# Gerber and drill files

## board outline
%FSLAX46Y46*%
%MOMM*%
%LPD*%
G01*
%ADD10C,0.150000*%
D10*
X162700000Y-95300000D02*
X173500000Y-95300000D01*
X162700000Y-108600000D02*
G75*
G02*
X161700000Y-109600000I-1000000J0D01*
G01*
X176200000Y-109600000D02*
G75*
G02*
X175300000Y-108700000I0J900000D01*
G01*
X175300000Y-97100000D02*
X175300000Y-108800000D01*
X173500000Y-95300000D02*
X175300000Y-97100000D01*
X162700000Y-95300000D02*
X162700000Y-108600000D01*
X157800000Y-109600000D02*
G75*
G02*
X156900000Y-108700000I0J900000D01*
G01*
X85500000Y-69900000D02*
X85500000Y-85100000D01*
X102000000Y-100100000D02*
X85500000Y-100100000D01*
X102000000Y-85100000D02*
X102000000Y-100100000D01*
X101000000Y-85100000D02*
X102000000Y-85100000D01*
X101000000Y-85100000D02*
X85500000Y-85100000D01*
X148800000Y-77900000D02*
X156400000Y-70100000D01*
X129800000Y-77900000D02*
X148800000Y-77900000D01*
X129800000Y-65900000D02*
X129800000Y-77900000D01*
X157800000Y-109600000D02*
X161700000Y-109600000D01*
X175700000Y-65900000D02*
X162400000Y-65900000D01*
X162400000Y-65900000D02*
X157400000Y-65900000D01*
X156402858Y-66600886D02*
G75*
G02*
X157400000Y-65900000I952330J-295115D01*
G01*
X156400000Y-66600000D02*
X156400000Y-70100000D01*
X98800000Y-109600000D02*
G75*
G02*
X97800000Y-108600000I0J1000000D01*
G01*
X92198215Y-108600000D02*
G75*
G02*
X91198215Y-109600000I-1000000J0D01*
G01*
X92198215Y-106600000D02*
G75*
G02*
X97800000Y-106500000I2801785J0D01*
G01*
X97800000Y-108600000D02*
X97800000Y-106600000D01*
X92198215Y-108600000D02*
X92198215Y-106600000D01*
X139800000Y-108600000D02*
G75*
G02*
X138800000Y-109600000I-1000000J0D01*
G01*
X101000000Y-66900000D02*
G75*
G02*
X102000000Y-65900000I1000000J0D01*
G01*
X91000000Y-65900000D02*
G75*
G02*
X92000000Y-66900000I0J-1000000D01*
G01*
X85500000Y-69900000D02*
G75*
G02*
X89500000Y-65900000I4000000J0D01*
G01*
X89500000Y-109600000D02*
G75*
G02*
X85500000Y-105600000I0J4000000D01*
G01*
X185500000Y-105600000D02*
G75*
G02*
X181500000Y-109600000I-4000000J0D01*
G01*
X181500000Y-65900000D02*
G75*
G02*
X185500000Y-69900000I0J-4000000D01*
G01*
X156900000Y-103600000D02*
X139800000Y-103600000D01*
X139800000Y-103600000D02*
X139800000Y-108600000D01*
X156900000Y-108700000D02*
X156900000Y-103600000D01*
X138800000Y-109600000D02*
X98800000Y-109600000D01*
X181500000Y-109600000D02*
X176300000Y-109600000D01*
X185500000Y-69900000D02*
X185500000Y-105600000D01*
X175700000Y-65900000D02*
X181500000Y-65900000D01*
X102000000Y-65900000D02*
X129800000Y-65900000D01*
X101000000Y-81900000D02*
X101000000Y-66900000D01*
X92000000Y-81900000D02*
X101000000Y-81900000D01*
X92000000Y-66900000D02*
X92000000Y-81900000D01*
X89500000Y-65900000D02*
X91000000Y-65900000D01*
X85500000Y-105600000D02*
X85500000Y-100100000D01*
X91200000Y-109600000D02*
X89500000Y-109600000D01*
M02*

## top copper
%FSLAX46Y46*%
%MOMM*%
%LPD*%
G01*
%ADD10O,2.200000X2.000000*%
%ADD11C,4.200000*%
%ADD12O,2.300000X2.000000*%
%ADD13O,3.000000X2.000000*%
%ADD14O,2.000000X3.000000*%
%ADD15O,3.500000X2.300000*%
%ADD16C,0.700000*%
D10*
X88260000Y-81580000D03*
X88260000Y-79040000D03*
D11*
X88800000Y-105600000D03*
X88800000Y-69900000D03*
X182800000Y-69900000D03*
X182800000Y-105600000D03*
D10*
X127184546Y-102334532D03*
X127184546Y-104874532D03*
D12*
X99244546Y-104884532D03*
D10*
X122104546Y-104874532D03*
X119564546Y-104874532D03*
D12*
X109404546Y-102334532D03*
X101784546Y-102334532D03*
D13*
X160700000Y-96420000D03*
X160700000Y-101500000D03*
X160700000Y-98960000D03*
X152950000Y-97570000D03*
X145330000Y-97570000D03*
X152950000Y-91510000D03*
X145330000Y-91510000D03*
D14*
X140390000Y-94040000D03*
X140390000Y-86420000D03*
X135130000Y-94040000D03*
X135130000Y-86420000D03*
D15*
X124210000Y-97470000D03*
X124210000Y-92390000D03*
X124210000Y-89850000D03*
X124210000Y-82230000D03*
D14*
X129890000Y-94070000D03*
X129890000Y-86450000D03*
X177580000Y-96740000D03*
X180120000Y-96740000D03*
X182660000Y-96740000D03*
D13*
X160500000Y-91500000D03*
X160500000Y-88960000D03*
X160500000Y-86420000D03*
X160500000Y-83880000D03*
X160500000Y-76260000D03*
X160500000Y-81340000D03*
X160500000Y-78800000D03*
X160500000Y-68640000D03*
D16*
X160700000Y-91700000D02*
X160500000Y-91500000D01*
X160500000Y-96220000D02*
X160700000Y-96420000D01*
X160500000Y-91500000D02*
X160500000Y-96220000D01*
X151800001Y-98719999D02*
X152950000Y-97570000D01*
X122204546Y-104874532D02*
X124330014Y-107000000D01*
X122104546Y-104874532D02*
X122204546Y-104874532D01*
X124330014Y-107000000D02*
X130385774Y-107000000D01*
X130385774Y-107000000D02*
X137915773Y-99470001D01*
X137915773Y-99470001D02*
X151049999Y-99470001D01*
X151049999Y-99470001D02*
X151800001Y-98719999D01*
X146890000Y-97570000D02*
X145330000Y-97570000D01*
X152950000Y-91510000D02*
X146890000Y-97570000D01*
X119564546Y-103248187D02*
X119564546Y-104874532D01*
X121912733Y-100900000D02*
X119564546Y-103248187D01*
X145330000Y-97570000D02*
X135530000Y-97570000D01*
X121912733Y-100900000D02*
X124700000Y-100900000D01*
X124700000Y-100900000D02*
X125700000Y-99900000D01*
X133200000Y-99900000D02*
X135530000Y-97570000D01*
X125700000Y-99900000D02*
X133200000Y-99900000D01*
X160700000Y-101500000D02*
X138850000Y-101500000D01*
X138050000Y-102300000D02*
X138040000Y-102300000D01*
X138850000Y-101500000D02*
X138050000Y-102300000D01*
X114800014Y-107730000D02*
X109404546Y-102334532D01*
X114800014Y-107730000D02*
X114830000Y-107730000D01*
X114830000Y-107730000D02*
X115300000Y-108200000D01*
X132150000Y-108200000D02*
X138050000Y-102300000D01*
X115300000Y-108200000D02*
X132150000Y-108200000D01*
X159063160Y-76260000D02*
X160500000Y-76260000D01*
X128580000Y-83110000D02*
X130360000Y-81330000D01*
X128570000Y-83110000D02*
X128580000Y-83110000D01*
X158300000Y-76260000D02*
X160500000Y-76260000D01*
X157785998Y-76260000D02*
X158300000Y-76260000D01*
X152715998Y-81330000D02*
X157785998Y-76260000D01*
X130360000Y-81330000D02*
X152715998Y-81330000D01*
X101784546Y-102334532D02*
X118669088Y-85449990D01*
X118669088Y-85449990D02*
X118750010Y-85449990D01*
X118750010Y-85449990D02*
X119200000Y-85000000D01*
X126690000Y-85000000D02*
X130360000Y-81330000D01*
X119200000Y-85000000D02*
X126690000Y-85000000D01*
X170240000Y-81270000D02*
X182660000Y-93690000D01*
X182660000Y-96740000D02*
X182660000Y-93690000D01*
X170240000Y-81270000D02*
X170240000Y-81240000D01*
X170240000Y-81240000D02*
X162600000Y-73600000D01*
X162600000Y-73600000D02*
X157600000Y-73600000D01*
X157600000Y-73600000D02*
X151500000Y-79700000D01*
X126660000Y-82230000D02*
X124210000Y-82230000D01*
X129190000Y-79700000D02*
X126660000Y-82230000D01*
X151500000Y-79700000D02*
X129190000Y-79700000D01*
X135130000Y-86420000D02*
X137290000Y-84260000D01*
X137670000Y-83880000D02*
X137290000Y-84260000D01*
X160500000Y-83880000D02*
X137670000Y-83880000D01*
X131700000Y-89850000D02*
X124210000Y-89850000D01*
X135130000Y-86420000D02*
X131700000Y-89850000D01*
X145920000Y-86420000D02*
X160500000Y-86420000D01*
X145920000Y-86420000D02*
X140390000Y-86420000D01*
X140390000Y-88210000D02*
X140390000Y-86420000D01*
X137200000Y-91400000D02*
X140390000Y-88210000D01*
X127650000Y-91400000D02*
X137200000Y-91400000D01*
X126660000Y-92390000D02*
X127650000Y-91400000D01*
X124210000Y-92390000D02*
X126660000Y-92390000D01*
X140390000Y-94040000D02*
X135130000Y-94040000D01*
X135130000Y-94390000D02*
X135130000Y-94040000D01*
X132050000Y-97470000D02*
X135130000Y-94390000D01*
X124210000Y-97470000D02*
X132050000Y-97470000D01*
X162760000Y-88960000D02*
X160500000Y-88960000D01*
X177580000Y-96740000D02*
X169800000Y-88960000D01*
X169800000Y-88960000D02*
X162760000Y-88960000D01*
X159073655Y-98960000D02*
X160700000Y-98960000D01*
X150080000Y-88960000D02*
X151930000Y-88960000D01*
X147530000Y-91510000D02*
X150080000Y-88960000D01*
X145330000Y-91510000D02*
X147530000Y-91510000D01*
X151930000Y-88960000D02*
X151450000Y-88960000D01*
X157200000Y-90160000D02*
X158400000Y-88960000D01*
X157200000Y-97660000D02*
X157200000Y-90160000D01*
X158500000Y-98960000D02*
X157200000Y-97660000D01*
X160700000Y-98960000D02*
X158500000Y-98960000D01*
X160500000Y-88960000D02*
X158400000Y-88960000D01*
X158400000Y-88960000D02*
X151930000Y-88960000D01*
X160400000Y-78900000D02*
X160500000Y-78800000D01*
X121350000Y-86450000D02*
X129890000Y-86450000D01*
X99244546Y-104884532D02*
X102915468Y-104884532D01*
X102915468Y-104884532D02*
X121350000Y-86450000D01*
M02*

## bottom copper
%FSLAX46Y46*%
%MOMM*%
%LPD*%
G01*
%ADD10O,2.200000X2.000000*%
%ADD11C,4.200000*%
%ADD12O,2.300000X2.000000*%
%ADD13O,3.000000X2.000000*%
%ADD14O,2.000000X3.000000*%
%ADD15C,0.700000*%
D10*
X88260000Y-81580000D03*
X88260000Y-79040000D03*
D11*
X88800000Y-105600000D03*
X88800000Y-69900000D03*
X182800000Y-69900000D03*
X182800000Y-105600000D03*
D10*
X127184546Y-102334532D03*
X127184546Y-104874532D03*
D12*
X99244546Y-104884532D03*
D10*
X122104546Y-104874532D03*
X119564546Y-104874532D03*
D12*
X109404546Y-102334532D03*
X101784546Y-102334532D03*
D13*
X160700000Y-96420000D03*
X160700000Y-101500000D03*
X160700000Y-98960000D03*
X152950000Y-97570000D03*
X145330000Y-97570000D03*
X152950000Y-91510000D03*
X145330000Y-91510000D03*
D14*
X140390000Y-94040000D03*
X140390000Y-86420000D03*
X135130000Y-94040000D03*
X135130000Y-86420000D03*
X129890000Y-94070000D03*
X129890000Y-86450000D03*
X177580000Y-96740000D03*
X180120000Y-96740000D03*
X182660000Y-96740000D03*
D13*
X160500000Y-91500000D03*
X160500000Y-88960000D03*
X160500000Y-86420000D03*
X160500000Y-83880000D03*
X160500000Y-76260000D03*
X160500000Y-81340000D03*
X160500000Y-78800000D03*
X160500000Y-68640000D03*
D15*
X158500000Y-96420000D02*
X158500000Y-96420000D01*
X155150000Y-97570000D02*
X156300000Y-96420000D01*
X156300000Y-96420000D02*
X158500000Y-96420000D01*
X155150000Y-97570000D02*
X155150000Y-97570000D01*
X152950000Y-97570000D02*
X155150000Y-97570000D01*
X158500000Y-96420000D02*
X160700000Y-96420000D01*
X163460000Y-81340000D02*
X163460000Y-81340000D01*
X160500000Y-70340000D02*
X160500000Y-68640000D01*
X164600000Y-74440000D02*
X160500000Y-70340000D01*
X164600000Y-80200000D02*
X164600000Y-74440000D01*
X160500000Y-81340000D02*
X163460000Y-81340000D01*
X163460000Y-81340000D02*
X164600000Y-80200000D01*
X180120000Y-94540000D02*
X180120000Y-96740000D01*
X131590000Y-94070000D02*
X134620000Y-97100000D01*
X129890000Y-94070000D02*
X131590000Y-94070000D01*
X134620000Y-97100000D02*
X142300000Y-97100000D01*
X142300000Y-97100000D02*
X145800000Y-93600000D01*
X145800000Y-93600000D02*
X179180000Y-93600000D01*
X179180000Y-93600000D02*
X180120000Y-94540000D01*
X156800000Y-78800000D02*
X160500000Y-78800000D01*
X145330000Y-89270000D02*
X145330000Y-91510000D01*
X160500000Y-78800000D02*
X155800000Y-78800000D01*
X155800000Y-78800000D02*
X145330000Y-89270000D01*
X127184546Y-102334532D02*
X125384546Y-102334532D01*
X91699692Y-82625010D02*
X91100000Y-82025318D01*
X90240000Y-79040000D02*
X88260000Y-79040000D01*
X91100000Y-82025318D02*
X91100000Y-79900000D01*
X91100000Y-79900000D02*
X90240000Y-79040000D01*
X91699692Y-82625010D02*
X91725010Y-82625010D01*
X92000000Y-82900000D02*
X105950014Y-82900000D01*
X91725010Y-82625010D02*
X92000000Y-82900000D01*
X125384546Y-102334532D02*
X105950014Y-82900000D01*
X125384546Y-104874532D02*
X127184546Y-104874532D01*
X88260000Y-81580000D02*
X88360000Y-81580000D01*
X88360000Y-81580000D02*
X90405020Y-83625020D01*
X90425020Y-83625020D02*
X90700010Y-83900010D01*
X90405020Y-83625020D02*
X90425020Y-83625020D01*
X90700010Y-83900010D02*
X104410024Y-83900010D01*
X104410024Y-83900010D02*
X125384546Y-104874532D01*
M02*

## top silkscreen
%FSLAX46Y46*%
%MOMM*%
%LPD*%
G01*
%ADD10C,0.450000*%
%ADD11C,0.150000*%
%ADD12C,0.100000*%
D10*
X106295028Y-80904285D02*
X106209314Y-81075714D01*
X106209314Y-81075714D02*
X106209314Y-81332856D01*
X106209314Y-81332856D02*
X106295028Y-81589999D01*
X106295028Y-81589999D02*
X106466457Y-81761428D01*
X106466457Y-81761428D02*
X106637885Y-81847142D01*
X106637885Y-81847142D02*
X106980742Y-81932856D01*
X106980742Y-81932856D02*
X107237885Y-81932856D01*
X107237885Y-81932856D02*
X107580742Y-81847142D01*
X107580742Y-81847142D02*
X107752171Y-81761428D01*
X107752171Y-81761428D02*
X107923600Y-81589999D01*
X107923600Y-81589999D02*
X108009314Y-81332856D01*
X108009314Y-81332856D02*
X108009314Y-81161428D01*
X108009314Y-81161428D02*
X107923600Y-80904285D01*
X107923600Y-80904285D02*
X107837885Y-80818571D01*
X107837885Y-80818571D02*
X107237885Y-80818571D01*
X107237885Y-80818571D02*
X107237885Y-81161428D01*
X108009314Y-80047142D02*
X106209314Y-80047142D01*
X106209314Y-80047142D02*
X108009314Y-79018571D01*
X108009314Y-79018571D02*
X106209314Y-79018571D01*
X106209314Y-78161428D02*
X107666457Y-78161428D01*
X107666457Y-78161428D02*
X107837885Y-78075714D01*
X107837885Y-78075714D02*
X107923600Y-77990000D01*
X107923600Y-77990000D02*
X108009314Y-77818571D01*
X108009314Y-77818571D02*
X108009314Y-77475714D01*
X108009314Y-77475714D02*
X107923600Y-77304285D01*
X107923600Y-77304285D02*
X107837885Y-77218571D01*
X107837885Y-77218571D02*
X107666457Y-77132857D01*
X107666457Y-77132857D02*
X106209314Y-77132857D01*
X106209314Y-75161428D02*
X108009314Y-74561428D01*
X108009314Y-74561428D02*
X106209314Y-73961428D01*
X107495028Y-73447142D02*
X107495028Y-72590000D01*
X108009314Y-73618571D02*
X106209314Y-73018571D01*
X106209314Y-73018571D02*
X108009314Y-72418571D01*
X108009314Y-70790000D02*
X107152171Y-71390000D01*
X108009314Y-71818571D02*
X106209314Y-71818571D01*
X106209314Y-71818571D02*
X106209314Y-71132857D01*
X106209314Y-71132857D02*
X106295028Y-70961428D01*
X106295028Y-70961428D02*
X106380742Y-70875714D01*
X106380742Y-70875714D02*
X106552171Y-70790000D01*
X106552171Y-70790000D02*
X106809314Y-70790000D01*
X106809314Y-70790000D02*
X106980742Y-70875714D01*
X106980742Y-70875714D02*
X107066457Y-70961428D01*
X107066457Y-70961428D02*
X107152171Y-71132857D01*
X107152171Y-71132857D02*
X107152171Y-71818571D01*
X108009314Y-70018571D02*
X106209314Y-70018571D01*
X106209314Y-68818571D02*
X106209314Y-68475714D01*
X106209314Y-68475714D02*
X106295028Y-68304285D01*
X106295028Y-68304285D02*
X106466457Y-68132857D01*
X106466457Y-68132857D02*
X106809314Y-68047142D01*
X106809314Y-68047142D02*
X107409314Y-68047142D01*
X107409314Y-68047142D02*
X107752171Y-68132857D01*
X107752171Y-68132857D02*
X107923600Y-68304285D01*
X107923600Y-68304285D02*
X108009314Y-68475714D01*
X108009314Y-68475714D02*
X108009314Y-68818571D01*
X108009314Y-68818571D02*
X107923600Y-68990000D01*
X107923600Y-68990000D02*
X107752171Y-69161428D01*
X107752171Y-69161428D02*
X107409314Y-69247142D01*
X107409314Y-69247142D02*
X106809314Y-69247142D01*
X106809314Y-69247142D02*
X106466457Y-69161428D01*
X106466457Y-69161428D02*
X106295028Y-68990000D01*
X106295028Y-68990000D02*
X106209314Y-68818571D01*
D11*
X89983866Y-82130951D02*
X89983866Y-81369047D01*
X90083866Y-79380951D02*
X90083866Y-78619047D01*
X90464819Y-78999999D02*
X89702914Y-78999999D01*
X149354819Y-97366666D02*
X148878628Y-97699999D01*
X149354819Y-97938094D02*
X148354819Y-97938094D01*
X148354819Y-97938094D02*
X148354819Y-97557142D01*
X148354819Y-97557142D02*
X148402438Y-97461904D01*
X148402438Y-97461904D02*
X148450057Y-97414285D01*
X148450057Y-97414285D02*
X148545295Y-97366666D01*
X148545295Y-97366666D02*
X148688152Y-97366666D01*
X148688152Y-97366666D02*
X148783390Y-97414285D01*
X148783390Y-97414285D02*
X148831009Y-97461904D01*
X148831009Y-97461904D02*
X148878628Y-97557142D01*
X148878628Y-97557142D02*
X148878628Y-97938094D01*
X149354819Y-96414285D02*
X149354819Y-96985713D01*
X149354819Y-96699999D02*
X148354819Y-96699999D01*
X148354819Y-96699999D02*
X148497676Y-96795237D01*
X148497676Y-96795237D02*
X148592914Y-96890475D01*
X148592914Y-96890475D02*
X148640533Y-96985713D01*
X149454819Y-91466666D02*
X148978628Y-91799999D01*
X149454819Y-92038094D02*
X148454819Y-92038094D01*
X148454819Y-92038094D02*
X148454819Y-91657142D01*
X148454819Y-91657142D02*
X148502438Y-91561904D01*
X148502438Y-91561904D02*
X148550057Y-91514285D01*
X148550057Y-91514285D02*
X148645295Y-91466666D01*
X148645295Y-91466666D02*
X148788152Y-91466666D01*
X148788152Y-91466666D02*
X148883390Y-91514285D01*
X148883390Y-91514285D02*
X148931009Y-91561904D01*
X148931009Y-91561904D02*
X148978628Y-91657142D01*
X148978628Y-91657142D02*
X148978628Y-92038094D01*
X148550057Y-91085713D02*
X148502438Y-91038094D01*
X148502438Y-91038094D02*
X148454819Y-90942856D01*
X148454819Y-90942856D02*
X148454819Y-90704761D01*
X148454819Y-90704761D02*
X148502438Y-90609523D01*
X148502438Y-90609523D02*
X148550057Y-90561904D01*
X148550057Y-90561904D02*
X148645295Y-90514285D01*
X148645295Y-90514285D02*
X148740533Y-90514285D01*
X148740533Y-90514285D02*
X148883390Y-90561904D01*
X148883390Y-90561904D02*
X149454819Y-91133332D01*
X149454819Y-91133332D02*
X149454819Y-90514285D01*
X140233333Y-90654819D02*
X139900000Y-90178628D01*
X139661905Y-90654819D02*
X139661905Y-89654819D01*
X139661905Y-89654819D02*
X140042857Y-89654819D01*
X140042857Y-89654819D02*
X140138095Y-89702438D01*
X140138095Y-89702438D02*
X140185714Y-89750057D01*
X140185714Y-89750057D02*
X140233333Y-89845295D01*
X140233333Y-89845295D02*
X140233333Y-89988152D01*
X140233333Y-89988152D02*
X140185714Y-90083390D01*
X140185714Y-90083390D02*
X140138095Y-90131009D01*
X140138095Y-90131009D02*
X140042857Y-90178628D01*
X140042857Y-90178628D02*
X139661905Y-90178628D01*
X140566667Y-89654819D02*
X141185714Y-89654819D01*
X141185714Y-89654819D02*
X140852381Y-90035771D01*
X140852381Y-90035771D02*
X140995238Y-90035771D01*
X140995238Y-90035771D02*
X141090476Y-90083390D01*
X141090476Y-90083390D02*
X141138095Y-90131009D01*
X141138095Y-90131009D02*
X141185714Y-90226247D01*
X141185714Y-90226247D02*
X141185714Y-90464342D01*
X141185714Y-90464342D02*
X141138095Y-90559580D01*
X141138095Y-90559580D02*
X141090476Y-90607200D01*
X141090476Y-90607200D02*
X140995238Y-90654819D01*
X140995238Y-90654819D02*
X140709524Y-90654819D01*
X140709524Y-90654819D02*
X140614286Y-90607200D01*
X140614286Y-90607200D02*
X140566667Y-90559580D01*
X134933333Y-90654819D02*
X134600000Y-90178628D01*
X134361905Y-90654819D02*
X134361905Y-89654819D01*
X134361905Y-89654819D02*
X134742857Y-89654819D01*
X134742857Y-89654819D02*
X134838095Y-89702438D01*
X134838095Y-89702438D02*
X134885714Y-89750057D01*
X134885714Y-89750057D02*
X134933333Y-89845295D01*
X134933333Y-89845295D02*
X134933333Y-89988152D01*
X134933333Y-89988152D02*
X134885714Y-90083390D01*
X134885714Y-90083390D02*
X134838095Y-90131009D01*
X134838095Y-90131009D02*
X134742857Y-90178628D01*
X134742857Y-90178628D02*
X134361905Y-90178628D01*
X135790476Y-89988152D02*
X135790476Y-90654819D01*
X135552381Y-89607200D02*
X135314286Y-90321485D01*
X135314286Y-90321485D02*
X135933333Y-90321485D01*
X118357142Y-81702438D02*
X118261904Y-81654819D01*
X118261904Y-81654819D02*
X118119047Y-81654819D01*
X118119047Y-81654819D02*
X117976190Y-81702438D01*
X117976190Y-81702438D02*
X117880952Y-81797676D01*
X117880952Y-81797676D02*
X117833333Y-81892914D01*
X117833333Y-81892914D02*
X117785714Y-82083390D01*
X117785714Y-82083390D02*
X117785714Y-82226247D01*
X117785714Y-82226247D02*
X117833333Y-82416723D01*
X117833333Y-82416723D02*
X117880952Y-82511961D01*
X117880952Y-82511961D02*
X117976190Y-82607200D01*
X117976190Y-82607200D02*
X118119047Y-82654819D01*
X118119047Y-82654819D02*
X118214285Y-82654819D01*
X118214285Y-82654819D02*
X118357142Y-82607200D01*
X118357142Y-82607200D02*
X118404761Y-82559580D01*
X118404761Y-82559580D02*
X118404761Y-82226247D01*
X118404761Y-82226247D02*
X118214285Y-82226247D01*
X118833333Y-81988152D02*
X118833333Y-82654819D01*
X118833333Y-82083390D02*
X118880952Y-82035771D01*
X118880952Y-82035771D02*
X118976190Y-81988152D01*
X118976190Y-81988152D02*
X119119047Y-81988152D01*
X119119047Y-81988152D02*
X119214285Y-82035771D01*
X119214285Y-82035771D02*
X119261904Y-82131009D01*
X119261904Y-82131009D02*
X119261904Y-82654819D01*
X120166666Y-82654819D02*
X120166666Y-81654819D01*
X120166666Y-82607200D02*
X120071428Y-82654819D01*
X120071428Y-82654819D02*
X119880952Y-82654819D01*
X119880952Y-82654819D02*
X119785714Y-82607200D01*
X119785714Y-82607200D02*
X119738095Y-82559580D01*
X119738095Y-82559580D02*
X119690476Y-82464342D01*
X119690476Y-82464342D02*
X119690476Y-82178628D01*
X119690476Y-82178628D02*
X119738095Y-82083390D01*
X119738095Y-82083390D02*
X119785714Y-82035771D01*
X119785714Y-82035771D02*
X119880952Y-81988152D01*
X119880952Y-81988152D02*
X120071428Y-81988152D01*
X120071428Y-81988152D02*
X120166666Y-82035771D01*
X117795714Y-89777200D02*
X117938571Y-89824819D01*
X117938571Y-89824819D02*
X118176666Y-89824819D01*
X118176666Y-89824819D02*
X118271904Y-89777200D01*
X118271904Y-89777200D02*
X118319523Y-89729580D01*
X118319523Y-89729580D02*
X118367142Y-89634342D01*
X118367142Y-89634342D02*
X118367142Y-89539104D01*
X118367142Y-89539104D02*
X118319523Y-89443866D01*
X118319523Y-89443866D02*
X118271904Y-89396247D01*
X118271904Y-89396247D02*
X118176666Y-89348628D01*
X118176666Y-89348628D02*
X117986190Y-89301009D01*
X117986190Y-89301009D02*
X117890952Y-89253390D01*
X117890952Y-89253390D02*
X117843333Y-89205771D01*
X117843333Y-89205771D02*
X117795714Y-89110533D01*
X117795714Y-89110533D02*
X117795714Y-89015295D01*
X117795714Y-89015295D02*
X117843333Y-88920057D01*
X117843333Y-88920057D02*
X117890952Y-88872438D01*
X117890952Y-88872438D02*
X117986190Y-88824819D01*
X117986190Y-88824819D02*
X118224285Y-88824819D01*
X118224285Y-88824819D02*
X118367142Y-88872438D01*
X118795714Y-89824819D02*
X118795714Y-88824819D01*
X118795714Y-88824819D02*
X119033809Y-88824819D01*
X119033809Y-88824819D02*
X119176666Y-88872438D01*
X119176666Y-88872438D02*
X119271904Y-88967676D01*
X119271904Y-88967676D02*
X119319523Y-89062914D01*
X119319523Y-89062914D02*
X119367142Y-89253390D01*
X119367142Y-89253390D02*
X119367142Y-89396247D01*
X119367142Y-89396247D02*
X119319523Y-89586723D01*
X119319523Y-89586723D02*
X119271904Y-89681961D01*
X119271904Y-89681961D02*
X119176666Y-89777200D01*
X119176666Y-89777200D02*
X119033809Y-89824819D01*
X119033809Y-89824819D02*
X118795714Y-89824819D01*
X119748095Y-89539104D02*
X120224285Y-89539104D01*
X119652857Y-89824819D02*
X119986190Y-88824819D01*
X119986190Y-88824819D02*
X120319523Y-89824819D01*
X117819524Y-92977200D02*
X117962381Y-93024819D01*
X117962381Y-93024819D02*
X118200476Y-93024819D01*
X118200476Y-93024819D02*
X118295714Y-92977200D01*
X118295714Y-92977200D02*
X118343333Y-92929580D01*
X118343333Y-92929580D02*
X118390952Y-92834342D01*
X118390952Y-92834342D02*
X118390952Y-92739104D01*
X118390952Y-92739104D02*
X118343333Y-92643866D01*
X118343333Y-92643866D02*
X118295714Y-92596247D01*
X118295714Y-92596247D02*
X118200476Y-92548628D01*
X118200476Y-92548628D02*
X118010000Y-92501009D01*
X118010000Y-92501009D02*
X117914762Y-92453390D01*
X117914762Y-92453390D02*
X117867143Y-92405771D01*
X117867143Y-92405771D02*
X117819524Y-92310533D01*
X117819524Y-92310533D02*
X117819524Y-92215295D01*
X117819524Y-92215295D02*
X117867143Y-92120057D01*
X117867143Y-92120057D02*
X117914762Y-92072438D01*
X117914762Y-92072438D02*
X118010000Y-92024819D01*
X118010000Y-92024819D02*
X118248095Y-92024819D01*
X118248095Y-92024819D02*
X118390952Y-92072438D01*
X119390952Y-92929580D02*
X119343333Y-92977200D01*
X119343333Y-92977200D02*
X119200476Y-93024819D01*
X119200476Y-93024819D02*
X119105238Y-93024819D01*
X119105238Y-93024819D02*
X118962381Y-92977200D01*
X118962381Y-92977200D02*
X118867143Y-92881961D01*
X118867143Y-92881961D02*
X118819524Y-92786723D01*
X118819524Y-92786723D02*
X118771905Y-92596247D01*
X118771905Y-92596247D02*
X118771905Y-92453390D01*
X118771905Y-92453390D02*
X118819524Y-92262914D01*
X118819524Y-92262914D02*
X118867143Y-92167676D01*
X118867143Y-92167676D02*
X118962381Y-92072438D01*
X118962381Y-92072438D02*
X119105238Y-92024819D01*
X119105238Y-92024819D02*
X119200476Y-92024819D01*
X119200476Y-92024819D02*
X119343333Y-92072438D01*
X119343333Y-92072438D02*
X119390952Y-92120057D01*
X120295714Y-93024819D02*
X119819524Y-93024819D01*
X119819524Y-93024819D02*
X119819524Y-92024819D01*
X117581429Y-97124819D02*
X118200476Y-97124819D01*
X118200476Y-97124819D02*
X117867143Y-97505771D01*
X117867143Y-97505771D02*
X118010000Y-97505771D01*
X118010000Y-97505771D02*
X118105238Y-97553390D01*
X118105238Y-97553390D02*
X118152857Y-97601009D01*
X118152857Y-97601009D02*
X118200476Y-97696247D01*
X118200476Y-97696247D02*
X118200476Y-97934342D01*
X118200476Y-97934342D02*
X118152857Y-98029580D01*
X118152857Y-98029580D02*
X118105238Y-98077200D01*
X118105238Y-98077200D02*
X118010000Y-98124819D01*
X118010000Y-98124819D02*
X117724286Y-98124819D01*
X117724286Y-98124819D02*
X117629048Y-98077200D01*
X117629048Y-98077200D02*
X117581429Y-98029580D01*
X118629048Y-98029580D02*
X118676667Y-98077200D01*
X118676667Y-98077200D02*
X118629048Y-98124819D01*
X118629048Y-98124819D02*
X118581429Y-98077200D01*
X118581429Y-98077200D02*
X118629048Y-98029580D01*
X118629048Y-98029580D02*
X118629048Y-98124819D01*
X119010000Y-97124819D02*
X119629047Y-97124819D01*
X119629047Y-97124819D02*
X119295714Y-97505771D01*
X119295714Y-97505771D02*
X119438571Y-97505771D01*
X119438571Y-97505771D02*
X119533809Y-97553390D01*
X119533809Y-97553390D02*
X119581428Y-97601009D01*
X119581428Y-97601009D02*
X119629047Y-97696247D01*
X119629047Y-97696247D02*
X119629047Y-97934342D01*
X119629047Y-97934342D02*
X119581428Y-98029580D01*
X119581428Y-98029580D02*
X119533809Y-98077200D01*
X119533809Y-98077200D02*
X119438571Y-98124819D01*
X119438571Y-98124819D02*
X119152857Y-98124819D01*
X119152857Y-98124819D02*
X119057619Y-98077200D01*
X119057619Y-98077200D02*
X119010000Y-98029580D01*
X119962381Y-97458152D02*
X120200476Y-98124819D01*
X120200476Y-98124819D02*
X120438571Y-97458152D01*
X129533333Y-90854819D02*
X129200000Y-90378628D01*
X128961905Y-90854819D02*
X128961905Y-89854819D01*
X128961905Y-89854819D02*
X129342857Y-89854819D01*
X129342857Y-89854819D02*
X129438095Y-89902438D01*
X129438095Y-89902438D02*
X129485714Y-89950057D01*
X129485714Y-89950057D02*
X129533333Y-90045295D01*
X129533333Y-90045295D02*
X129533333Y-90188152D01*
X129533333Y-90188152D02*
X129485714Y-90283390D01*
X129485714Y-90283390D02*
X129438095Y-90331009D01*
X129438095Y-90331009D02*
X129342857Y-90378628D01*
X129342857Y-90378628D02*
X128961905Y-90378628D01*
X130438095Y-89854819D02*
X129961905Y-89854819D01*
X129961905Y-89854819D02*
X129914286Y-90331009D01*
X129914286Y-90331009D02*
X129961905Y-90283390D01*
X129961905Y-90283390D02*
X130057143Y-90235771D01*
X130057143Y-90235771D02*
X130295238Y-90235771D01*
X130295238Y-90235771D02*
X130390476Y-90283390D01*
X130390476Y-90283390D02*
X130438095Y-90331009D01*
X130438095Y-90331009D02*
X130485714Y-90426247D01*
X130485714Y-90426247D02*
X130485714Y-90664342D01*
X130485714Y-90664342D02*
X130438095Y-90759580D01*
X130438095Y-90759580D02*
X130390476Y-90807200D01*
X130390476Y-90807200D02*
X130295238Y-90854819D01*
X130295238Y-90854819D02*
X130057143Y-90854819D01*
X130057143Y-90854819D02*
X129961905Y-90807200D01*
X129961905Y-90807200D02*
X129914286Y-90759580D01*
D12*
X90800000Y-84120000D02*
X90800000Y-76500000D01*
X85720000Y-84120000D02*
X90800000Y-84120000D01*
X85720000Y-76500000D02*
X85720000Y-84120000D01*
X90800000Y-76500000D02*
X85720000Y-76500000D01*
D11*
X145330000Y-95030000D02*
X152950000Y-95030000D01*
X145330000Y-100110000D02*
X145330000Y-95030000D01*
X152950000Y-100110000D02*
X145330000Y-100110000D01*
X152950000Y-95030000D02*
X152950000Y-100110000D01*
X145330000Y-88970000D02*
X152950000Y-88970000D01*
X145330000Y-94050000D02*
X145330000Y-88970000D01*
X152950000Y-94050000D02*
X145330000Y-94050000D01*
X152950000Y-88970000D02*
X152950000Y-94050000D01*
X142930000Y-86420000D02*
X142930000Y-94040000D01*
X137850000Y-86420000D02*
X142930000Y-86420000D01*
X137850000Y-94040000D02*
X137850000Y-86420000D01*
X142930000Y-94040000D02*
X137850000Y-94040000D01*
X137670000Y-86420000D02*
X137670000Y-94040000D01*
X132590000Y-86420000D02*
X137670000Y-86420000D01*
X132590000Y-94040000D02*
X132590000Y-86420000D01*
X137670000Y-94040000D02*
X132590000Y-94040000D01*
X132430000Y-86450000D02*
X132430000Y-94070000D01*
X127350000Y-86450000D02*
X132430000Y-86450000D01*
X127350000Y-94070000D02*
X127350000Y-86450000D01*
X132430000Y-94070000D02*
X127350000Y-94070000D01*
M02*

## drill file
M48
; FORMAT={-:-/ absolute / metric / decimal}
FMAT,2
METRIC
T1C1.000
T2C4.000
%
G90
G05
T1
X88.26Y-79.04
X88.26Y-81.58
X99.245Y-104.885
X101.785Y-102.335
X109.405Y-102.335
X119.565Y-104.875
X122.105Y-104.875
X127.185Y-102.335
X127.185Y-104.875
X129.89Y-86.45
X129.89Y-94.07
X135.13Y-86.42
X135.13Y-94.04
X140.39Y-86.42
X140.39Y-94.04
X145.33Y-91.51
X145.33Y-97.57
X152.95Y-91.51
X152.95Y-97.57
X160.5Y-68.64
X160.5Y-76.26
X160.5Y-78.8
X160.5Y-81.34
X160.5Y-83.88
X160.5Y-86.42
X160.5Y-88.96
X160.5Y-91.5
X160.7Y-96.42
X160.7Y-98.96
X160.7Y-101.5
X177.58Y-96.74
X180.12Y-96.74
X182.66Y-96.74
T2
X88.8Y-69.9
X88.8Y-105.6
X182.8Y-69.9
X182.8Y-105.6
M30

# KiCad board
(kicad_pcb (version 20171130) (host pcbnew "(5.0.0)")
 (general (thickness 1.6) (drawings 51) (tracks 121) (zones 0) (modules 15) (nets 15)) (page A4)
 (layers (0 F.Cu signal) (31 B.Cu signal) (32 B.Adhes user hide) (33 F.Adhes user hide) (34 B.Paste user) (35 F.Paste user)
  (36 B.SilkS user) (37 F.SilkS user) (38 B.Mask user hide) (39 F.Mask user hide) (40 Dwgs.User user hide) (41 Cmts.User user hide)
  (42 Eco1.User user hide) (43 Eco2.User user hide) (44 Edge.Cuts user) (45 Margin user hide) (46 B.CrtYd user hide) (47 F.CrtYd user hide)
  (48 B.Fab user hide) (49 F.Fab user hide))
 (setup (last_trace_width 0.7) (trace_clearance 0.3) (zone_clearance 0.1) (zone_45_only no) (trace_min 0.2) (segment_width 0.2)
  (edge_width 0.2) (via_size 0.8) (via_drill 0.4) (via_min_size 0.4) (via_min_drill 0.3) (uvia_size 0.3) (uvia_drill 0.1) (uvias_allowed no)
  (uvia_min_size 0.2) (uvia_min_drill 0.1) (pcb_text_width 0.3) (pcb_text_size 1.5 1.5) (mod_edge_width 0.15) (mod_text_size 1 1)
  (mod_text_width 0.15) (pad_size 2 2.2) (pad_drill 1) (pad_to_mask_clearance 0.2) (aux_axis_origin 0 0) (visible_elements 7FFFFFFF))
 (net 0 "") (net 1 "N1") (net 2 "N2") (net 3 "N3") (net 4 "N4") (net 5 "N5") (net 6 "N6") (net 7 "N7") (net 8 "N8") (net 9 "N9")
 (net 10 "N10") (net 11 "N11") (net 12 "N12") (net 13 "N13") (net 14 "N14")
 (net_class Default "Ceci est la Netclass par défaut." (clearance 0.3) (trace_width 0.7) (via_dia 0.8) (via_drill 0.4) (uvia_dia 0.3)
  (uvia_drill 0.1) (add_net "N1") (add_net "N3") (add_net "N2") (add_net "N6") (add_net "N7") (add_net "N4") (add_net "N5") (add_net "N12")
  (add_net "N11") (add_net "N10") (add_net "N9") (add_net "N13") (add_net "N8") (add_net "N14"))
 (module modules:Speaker (layer B.Cu) (at 90.8 76.5 270)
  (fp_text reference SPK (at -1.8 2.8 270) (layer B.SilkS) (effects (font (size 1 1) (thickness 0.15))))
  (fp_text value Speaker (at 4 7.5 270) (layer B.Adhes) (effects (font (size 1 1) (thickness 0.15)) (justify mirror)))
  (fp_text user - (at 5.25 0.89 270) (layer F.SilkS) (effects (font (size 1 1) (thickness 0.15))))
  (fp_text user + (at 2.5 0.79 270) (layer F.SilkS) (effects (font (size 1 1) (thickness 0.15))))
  (fp_line (start 7.62 0) (end 0 0) (layer F.SilkS) (width 0.1))
  (fp_line (start 7.62 5.08) (end 7.62 0) (layer F.SilkS) (width 0.1))
  (fp_line (start 0 5.08) (end 7.62 5.08) (layer F.SilkS) (width 0.1))
  (fp_line (start 0 0) (end 0 5.08) (layer F.SilkS) (width 0.1))
  (pad 2 thru_hole oval (at 5.08 2.54 270) (size 2 2.2) (drill 1) (layers *.Cu *.Paste *.Mask) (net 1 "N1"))
  (pad 1 thru_hole oval (at 2.54 2.54 270) (size 2 2.2) (drill 1) (layers *.Cu *.Paste *.Mask) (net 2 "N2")))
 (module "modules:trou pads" (layer F.Cu) (at 88.8 105.6)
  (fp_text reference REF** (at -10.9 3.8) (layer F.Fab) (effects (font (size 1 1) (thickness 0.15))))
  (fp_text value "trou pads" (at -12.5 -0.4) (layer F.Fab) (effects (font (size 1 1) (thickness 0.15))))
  (pad "" np_thru_hole circle (at 0 0) (size 4.2 4.2) (drill 4) (layers *.Cu *.Mask)))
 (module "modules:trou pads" (layer F.Cu) (at 88.8 69.9)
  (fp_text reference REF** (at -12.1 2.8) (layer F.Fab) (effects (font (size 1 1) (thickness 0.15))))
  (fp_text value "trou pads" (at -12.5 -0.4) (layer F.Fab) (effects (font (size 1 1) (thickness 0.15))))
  (pad "" np_thru_hole circle (at 0 0) (size 4.2 4.2) (drill 4) (layers *.Cu *.Mask)))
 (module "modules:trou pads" (layer F.Cu) (at 182.8 69.9)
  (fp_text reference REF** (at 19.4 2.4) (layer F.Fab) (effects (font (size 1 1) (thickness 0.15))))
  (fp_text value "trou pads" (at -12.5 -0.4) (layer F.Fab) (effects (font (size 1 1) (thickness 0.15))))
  (pad "" np_thru_hole circle (at 0 0) (size 4.2 4.2) (drill 4) (layers *.Cu *.Mask)))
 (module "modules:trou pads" (layer F.Cu) (at 182.8 105.6)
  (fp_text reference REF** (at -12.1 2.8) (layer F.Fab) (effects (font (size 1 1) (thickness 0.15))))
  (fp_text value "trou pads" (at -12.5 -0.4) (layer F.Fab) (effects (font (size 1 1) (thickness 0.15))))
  (pad "" np_thru_hole circle (at 0 0) (size 4.2 4.2) (drill 4) (layers *.Cu *.Mask)))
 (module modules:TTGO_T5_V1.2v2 (layer F.Cu) (at 127.734546 102.554532 90)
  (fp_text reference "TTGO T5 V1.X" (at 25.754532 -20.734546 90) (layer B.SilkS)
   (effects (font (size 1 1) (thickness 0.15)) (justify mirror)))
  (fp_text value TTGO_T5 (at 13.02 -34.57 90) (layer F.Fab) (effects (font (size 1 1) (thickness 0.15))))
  (pad "HP +" thru_hole oval (at 0.22 -0.55 90) (size 2 2.2) (drill 1) (layers *.Cu *.Paste *.Mask) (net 2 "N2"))
  (pad "HP -" thru_hole oval (at -2.32 -0.55 90) (size 2 2.2) (drill 1) (layers *.Cu *.Paste *.Mask) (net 1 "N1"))
  (pad 12 thru_hole oval (at -2.33 -28.49 90) (size 2 2.3) (drill 1) (layers *.Cu *.Paste *.Mask) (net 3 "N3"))
  (pad 3 thru_hole oval (at -2.32 -5.63 90) (size 2 2.2) (drill 1) (layers *.Cu *.Paste *.Mask) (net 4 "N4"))
  (pad 4 thru_hole oval (at -2.32 -8.17 90) (size 2 2.2) (drill 1) (layers *.Cu *.Paste *.Mask) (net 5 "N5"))
  (pad 20 thru_hole oval (at 0.22 -18.33 90) (size 2 2.3) (drill 1) (layers *.Cu *.Paste *.Mask) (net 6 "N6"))
  (pad 23 thru_hole oval (at 0.22 -25.95 90) (size 2 2.3) (drill 1) (layers *.Cu *.Paste *.Mask) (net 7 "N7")))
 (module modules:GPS (layer F.Cu) (at 160.7 96.42 270)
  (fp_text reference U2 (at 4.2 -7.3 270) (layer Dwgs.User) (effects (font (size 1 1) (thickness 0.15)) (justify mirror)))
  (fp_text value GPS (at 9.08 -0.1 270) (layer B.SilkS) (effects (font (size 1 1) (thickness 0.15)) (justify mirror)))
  (pad 1 thru_hole oval (at 0 0 270) (size 2 3) (drill 1) (layers *.Cu *.Paste *.Mask) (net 4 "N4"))
  (pad 3 thru_hole oval (at 5.08 0 270) (size 2 3) (drill 1) (layers *.Cu *.Paste *.Mask) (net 6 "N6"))
  (pad 2 thru_hole oval (at 2.54 0 270) (size 2 3) (drill 1) (layers *.Cu *.Paste *.Mask) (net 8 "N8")))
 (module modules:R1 (layer F.Cu) (at 145.33 97.57 270)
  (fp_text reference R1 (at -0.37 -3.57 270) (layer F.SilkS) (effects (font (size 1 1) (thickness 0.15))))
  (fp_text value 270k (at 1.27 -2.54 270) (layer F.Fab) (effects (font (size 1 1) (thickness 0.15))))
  (fp_line (start -2.54 0) (end -2.54 -7.62) (layer F.SilkS) (width 0.15))
  (fp_line (start 2.54 0) (end -2.54 0) (layer F.SilkS) (width 0.15))
  (fp_line (start 2.54 -7.62) (end 2.54 0) (layer F.SilkS) (width 0.15))
  (fp_line (start -2.54 -7.62) (end 2.54 -7.62) (layer F.SilkS) (width 0.15))
  (pad 2 thru_hole oval (at 0 -7.62 270) (size 2 3) (drill 1) (layers *.Cu *.Paste *.Mask) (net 4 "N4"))
  (pad 1 thru_hole oval (at 0 0 270) (size 2 3) (drill 1) (layers *.Cu *.Paste *.Mask) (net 5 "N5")))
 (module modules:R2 (layer F.Cu) (at 145.33 91.51 270)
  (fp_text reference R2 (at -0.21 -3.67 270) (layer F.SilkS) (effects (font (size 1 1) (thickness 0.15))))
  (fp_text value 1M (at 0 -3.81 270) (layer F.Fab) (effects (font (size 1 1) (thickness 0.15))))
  (fp_line (start -2.54 0) (end -2.54 -7.62) (layer F.SilkS) (width 0.15))
  (fp_line (start 2.54 0) (end -2.54 0) (layer F.SilkS) (width 0.15))
  (fp_line (start 2.54 -7.62) (end 2.54 0) (layer F.SilkS) (width 0.15))
  (fp_line (start -2.54 -7.62) (end 2.54 -7.62) (layer F.SilkS) (width 0.15))
  (pad 2 thru_hole oval (at 0 -7.62 270) (size 2 3) (drill 1) (layers *.Cu *.Paste *.Mask) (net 5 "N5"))
  (pad 1 thru_hole oval (at 0 0 270) (size 2 3) (drill 1) (layers *.Cu *.Paste *.Mask) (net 8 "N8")))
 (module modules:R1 (layer F.Cu) (at 140.39 86.42 180)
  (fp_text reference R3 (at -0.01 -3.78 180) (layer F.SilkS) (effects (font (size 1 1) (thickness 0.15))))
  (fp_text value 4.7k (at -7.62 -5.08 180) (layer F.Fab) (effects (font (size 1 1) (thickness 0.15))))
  (fp_line (start -2.54 0) (end -2.54 -7.62) (layer F.SilkS) (width 0.15))
  (fp_line (start 2.54 0) (end -2.54 0) (layer F.SilkS) (width 0.15))
  (fp_line (start 2.54 -7.62) (end 2.54 0) (layer F.SilkS) (width 0.15))
  (fp_line (start -2.54 -7.62) (end 2.54 -7.62) (layer F.SilkS) (width 0.15))
  (pad 2 thru_hole oval (at 0 -7.62 180) (size 2 3) (drill 1) (layers *.Cu *.Paste *.Mask) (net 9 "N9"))
  (pad 1 thru_hole oval (at 0 0 180) (size 2 3) (drill 1) (layers *.Cu *.Paste *.Mask) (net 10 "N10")))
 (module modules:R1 (layer F.Cu) (at 135.13 86.42 180)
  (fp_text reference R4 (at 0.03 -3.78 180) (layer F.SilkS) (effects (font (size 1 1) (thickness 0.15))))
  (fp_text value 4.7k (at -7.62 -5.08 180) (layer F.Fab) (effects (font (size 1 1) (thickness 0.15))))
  (fp_line (start -2.54 0) (end -2.54 -7.62) (layer F.SilkS) (width 0.15))
  (fp_line (start 2.54 0) (end -2.54 0) (layer F.SilkS) (width 0.15))
  (fp_line (start 2.54 -7.62) (end 2.54 0) (layer F.SilkS) (width 0.15))
  (fp_line (start -2.54 -7.62) (end 2.54 -7.62) (layer F.SilkS) (width 0.15))
  (pad 2 thru_hole oval (at 0 -7.62 180) (size 2 3) (drill 1) (layers *.Cu *.Paste *.Mask) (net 9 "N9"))
  (pad 1 thru_hole oval (at 0 0 180) (size 2 3) (drill 1) (layers *.Cu *.Paste *.Mask) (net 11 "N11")))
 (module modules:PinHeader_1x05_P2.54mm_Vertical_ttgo (layer F.Cu) (at 124.21 84.77)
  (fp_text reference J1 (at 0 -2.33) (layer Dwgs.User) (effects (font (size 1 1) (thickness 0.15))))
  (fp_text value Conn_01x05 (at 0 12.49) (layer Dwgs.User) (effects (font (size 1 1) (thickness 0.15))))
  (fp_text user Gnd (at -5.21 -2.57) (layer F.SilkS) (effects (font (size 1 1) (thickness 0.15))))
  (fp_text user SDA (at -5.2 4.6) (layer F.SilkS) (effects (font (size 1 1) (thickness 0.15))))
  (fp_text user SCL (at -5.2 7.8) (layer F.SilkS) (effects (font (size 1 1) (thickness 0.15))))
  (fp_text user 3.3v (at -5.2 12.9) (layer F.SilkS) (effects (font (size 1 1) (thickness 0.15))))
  (pad 5 smd oval (at 0 12.7) (size 3.5 2.3) (layers F.Cu F.Paste F.Mask) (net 9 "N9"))
  (pad 4 smd oval (at 0 7.62) (size 3.5 2.3) (layers F.Cu F.Paste F.Mask) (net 10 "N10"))
  (pad 3 smd oval (at 0 5.08) (size 3.5 2.3) (layers F.Cu F.Paste F.Mask) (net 11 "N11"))
  (pad 1 smd oval (at 0 -2.54) (size 3.5 2.3) (layers F.Cu F.Paste F.Mask) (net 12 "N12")))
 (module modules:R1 (layer F.Cu) (at 129.89 86.45 180)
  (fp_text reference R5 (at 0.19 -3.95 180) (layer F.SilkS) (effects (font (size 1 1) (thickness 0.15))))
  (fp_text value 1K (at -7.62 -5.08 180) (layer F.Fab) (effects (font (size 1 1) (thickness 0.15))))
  (fp_line (start -2.54 0) (end -2.54 -7.62) (layer F.SilkS) (width 0.15))
  (fp_line (start 2.54 0) (end -2.54 0) (layer F.SilkS) (width 0.15))
  (fp_line (start 2.54 -7.62) (end 2.54 0) (layer F.SilkS) (width 0.15))
  (fp_line (start -2.54 -7.62) (end 2.54 -7.62) (layer F.SilkS) (width 0.15))
  (pad 2 thru_hole oval (at 0 -7.62 180) (size 2 3) (drill 1) (layers *.Cu *.Paste *.Mask) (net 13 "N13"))
  (pad 1 thru_hole oval (at 0 0 180) (size 2 3) (drill 1) (layers *.Cu *.Paste *.Mask) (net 3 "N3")))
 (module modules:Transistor (layer F.Cu) (at 185.2 94.2 180)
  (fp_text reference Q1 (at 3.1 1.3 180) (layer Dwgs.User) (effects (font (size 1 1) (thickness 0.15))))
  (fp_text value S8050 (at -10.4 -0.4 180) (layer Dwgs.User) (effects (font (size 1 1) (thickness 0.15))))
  (pad 3 thru_hole oval (at 7.62 -2.54 180) (size 2 3) (drill 1) (layers *.Cu *.Paste *.Mask) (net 8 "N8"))
  (pad 2 thru_hole oval (at 5.08 -2.54 180) (size 2 3) (drill 1) (layers *.Cu *.Paste *.Mask) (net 13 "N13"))
  (pad 1 thru_hole oval (at 2.54 -2.54 180) (size 2 3) (drill 1) (layers *.Cu *.Paste *.Mask) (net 12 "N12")))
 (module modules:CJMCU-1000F (layer B.Cu) (at 163.04 78.8 270)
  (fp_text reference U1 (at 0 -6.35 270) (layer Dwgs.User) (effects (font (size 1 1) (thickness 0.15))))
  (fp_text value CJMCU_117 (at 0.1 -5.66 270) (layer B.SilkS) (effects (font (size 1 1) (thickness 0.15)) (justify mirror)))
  (pad 1 thru_hole oval (at 12.7 2.54 270) (size 2 3) (drill 1) (layers *.Cu *.Paste *.Mask) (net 4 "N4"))
  (pad 2 thru_hole oval (at 10.16 2.54 270) (size 2 3) (drill 1) (layers *.Cu *.Paste *.Mask) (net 8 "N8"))
  (pad 3 thru_hole oval (at 7.62 2.54 270) (size 2 3) (drill 1) (layers *.Cu *.Paste *.Mask) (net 10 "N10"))
  (pad 4 thru_hole oval (at 5.08 2.54 270) (size 2 3) (drill 1) (layers *.Cu *.Paste *.Mask) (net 11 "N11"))
  (pad 7 thru_hole oval (at -2.54 2.54 270) (size 2 3) (drill 1) (layers *.Cu *.Paste *.Mask) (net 7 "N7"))
  (pad 5 thru_hole oval (at 2.54 2.54 270) (size 2 3) (drill 1) (layers *.Cu *.Paste *.Mask) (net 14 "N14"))
  (pad 6 thru_hole oval (at 0 2.54 270) (size 2 3) (drill 1) (layers *.Cu *.Paste *.Mask) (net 8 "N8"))
  (pad 10 thru_hole oval (at -10.16 2.54 270) (size 2 3) (drill 1) (layers *.Cu *.Paste *.Mask) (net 14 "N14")))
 (gr_line (start 162.7 95.3) (end 173.5 95.3) (layer Edge.Cuts) (width 0.15))
 (gr_arc (start 161.7 108.6) (end 161.7 109.6) (angle -90) (layer Edge.Cuts) (width 0.15))
 (gr_arc (start 176.2 108.7) (end 175.3 108.7) (angle -90) (layer Edge.Cuts) (width 0.15))
 (gr_line (start 175.3 97.1) (end 175.3 108.8) (layer Edge.Cuts) (width 0.15))
 (gr_line (start 173.5 95.3) (end 175.3 97.1) (layer Edge.Cuts) (width 0.15))
 (gr_line (start 162.7 95.3) (end 162.7 108.6) (layer Edge.Cuts) (width 0.15))
 (gr_arc (start 157.8 108.7) (end 156.9 108.7) (angle -90) (layer Edge.Cuts) (width 0.15))
 (gr_line (start 85.5 69.9) (end 85.5 85.1) (layer Edge.Cuts) (width 0.15))
 (gr_line (start 102 100.1) (end 85.5 100.1) (layer Edge.Cuts) (width 0.15))
 (gr_line (start 102 85.1) (end 102 100.1) (layer Edge.Cuts) (width 0.15))
 (gr_line (start 101 85.1) (end 102 85.1) (layer Edge.Cuts) (width 0.15))
 (gr_line (start 101 85.1) (end 85.5 85.1) (layer Edge.Cuts) (width 0.15))
 (gr_line (start 148.8 77.9) (end 156.4 70.1) (layer Edge.Cuts) (width 0.15))
 (gr_line (start 129.8 77.9) (end 148.8 77.9) (layer Edge.Cuts) (width 0.15))
 (gr_line (start 129.8 65.9) (end 129.8 77.9) (layer Edge.Cuts) (width 0.15))
 (gr_line (start 157.8 109.6) (end 161.7 109.6) (layer Edge.Cuts) (width 0.15))
 (gr_line (start 175.7 65.9) (end 162.4 65.9) (layer Edge.Cuts) (width 0.15))
 (gr_line (start 162.4 65.9) (end 157.4 65.9) (layer Edge.Cuts) (width 0.15))
 (gr_arc (start 157.355188 66.896001) (end 157.4 65.9) (angle -75.35856355) (layer Edge.Cuts) (width 0.15))
 (gr_line (start 156.4 66.6) (end 156.4 70.1) (layer Edge.Cuts) (width 0.15))
 (gr_arc (start 98.8 108.6) (end 97.8 108.6) (angle -90) (layer Edge.Cuts) (width 0.15))
 (gr_arc (start 91.198215 108.6) (end 91.198215 109.6) (angle -90) (layer Edge.Cuts) (width 0.15))
 (gr_arc (start 95 106.6) (end 97.8 106.5) (angle -177.9545915) (layer Edge.Cuts) (width 0.15))
 (gr_line (start 97.8 108.6) (end 97.8 106.6) (layer Edge.Cuts) (width 0.15))
 (gr_line (start 92.198215 108.6) (end 92.198215 106.6) (layer Edge.Cuts) (width 0.15))
 (gr_arc (start 138.8 108.6) (end 138.8 109.6) (angle -90) (layer Edge.Cuts) (width 0.15))
 (gr_arc (start 102 66.9) (end 102 65.9) (angle -90) (layer Edge.Cuts) (width 0.15))
 (gr_arc (start 91 66.9) (end 92 66.9) (angle -90) (layer Edge.Cuts) (width 0.15))
 (gr_arc (start 89.5 69.9) (end 89.5 65.9) (angle -90) (layer Edge.Cuts) (width 0.15))
 (gr_arc (start 89.5 105.6) (end 85.5 105.6) (angle -90) (layer Edge.Cuts) (width 0.15))
 (gr_arc (start 181.5 105.6) (end 181.5 109.6) (angle -90) (layer Edge.Cuts) (width 0.15))
 (gr_arc (start 181.5 69.9) (end 185.5 69.9) (angle -90) (layer Edge.Cuts) (width 0.15))
 (gr_line (start 156.9 103.6) (end 139.8 103.6) (layer Edge.Cuts) (width 0.15))
 (gr_line (start 139.8 103.6) (end 139.8 108.6) (layer Edge.Cuts) (width 0.15))
 (gr_line (start 156.9 108.7) (end 156.9 103.6) (layer Edge.Cuts) (width 0.15))
 (gr_line (start 138.8 109.6) (end 98.8 109.6) (layer Edge.Cuts) (width 0.15))
 (gr_line (start 181.5 109.6) (end 176.3 109.6) (layer Edge.Cuts) (width 0.15))
 (gr_line (start 185.5 69.9) (end 185.5 105.6) (layer Edge.Cuts) (width 0.15))
 (gr_line (start 175.7 65.9) (end 181.5 65.9) (layer Edge.Cuts) (width 0.15))
 (gr_line (start 102 65.9) (end 129.8 65.9) (layer Edge.Cuts) (width 0.15))
 (gr_line (start 101 81.9) (end 101 66.9) (layer Edge.Cuts) (width 0.15))
 (gr_line (start 92 81.9) (end 101 81.9) (layer Edge.Cuts) (width 0.15))
 (gr_line (start 92 66.9) (end 92 81.9) (layer Edge.Cuts) (width 0.15))
 (gr_line (start 89.5 65.9) (end 91 65.9) (layer Edge.Cuts) (width 0.15))
 (gr_line (start 85.5 105.6) (end 85.5 100.1) (layer Edge.Cuts) (width 0.15))
 (gr_line (start 91.2 109.6) (end 89.5 109.6) (layer Edge.Cuts) (width 0.15))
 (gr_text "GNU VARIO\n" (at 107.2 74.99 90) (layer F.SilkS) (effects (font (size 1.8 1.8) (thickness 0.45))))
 (segment (start 160.7 91.7) (end 160.5 91.5) (width 0.7) (layer F.Cu) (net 4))
 (segment (start 160.5 96.22) (end 160.7 96.42) (width 0.7) (layer F.Cu) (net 4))
 (segment (start 160.5 91.5) (end 160.5 96.22) (width 0.7) (layer F.Cu) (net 4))
 (segment (start 158.5 96.42) (end 158.5 96.42) (width 0.7) (layer B.Cu) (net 4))
 (segment (start 155.15 97.57) (end 156.3 96.42) (width 0.7) (layer B.Cu) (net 4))
 (segment (start 156.3 96.42) (end 158.5 96.42) (width 0.7) (layer B.Cu) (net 4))
 (segment (start 155.15 97.57) (end 155.15 97.57) (width 0.7) (layer B.Cu) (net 4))
 (segment (start 152.95 97.57) (end 155.15 97.57) (width 0.7) (layer B.Cu) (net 4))
 (segment (start 158.5 96.42) (end 160.7 96.42) (width 0.7) (layer B.Cu) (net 4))
 (segment (start 151.800001 98.719999) (end 152.95 97.57) (width 0.7) (layer F.Cu) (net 4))
 (segment (start 122.204546 104.874532) (end 124.330014 107) (width 0.7) (layer F.Cu) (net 4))
 (segment (start 122.104546 104.874532) (end 122.204546 104.874532) (width 0.7) (layer F.Cu) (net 4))
 (segment (start 124.330014 107) (end 130.385774 107) (width 0.7) (layer F.Cu) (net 4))
 (segment (start 130.385774 107) (end 137.915773 99.470001) (width 0.7) (layer F.Cu) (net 4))
 (segment (start 137.915773 99.470001) (end 151.049999 99.470001) (width 0.7) (layer F.Cu) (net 4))
 (segment (start 151.049999 99.470001) (end 151.800001 98.719999) (width 0.7) (layer F.Cu) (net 4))
 (segment (start 146.89 97.57) (end 145.33 97.57) (width 0.7) (layer F.Cu) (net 5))
 (segment (start 152.95 91.51) (end 146.89 97.57) (width 0.7) (layer F.Cu) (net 5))
 (segment (start 119.564546 103.248187) (end 119.564546 104.874532) (width 0.7) (layer F.Cu) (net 5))
 (segment (start 121.912733 100.9) (end 119.564546 103.248187) (width 0.7) (layer F.Cu) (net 5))
 (segment (start 145.33 97.57) (end 135.53 97.57) (width 0.7) (layer F.Cu) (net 5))
 (segment (start 121.912733 100.9) (end 124.7 100.9) (width 0.7) (layer F.Cu) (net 5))
 (segment (start 124.7 100.9) (end 125.7 99.9) (width 0.7) (layer F.Cu) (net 5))
 (segment (start 133.2 99.9) (end 135.53 97.57) (width 0.7) (layer F.Cu) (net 5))
 (segment (start 125.7 99.9) (end 133.2 99.9) (width 0.7) (layer F.Cu) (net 5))
 (segment (start 160.7 101.5) (end 138.85 101.5) (width 0.7) (layer F.Cu) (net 6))
 (segment (start 138.05 102.3) (end 138.04 102.3) (width 0.7) (layer F.Cu) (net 6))
 (segment (start 138.85 101.5) (end 138.05 102.3) (width 0.7) (layer F.Cu) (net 6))
 (segment (start 114.800014 107.73) (end 109.404546 102.334532) (width 0.7) (layer F.Cu) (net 6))
 (segment (start 114.800014 107.73) (end 114.83 107.73) (width 0.7) (layer F.Cu) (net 6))
 (segment (start 114.83 107.73) (end 115.3 108.2) (width 0.7) (layer F.Cu) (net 6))
 (segment (start 132.15 108.2) (end 138.05 102.3) (width 0.7) (layer F.Cu) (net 6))
 (segment (start 115.3 108.2) (end 132.15 108.2) (width 0.7) (layer F.Cu) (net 6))
 (segment (start 159.06316 76.26) (end 160.5 76.26) (width 0.7) (layer F.Cu) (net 7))
 (segment (start 128.58 83.11) (end 130.36 81.33) (width 0.7) (layer F.Cu) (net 7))
 (segment (start 128.57 83.11) (end 128.58 83.11) (width 0.7) (layer F.Cu) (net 7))
 (segment (start 158.3 76.26) (end 160.5 76.26) (width 0.7) (layer F.Cu) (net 7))
 (segment (start 157.785998 76.26) (end 158.3 76.26) (width 0.7) (layer F.Cu) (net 7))
 (segment (start 152.715998 81.33) (end 157.785998 76.26) (width 0.7) (layer F.Cu) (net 7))
 (segment (start 130.36 81.33) (end 152.715998 81.33) (width 0.7) (layer F.Cu) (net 7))
 (segment (start 101.784546 102.334532) (end 118.669088 85.44999) (width 0.7) (layer F.Cu) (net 7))
 (segment (start 118.669088 85.44999) (end 118.75001 85.44999) (width 0.7) (layer F.Cu) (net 7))
 (segment (start 118.75001 85.44999) (end 119.2 85) (width 0.7) (layer F.Cu) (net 7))
 (segment (start 126.69 85) (end 130.36 81.33) (width 0.7) (layer F.Cu) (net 7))
 (segment (start 119.2 85) (end 126.69 85) (width 0.7) (layer F.Cu) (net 7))
 (segment (start 163.46 81.34) (end 163.46 81.34) (width 0.7) (layer B.Cu) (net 14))
 (segment (start 160.5 70.34) (end 160.5 68.64) (width 0.7) (layer B.Cu) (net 14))
 (segment (start 164.6 74.44) (end 160.5 70.34) (width 0.7) (layer B.Cu) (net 14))
 (segment (start 164.6 80.2) (end 164.6 74.44) (width 0.7) (layer B.Cu) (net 14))
 (segment (start 160.5 81.34) (end 163.46 81.34) (width 0.7) (layer B.Cu) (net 14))
 (segment (start 163.46 81.34) (end 164.6 80.2) (width 0.7) (layer B.Cu) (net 14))
 (segment (start 170.24 81.27) (end 182.66 93.69) (width 0.7) (layer F.Cu) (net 12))
 (segment (start 182.66 96.74) (end 182.66 93.69) (width 0.7) (layer F.Cu) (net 12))
 (segment (start 170.24 81.27) (end 170.24 81.24) (width 0.7) (layer F.Cu) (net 12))
 (segment (start 170.24 81.24) (end 162.6 73.6) (width 0.7) (layer F.Cu) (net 12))
 (segment (start 162.6 73.6) (end 157.6 73.6) (width 0.7) (layer F.Cu) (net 12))
 (segment (start 157.6 73.6) (end 151.5 79.7) (width 0.7) (layer F.Cu) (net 12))
 (segment (start 126.66 82.23) (end 124.21 82.23) (width 0.7) (layer F.Cu) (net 12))
 (segment (start 129.19 79.7) (end 126.66 82.23) (width 0.7) (layer F.Cu) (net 12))
 (segment (start 151.5 79.7) (end 129.19 79.7) (width 0.7) (layer F.Cu) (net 12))
 (segment (start 135.13 86.42) (end 137.29 84.26) (width 0.7) (layer F.Cu) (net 11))
 (segment (start 137.67 83.88) (end 137.29 84.26) (width 0.7) (layer F.Cu) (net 11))
 (segment (start 160.5 83.88) (end 137.67 83.88) (width 0.7) (layer F.Cu) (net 11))
 (segment (start 131.7 89.85) (end 124.21 89.85) (width 0.7) (layer F.Cu) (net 11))
 (segment (start 135.13 86.42) (end 131.7 89.85) (width 0.7) (layer F.Cu) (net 11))
 (segment (start 145.92 86.42) (end 160.5 86.42) (width 0.7) (layer F.Cu) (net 10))
 (segment (start 145.92 86.42) (end 140.39 86.42) (width 0.7) (layer F.Cu) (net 10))
 (segment (start 140.39 88.21) (end 140.39 86.42) (width 0.7) (layer F.Cu) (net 10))
 (segment (start 137.2 91.4) (end 140.39 88.21) (width 0.7) (layer F.Cu) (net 10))
 (segment (start 127.65 91.4) (end 137.2 91.4) (width 0.7) (layer F.Cu) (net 10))
 (segment (start 126.66 92.39) (end 127.65 91.4) (width 0.7) (layer F.Cu) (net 10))
 (segment (start 124.21 92.39) (end 126.66 92.39) (width 0.7) (layer F.Cu) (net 10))
 (segment (start 140.39 94.04) (end 135.13 94.04) (width 0.7) (layer F.Cu) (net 9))
 (segment (start 135.13 94.39) (end 135.13 94.04) (width 0.7) (layer F.Cu) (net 9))
 (segment (start 132.05 97.47) (end 135.13 94.39) (width 0.7) (layer F.Cu) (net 9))
 (segment (start 124.21 97.47) (end 132.05 97.47) (width 0.7) (layer F.Cu) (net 9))
 (segment (start 180.12 94.54) (end 180.12 96.74) (width 0.7) (layer B.Cu) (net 13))
 (segment (start 131.59 94.07) (end 134.62 97.1) (width 0.7) (layer B.Cu) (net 13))
 (segment (start 129.89 94.07) (end 131.59 94.07) (width 0.7) (layer B.Cu) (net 13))
 (segment (start 134.62 97.1) (end 142.3 97.1) (width 0.7) (layer B.Cu) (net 13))
 (segment (start 142.3 97.1) (end 145.8 93.6) (width 0.7) (layer B.Cu) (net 13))
 (segment (start 145.8 93.6) (end 179.18 93.6) (width 0.7) (layer B.Cu) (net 13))
 (segment (start 179.18 93.6) (end 180.12 94.54) (width 0.7) (layer B.Cu) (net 13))
 (segment (start 162.76 88.96) (end 160.5 88.96) (width 0.7) (layer F.Cu) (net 8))
 (segment (start 177.58 96.74) (end 169.8 88.96) (width 0.7) (layer F.Cu) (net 8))
 (segment (start 169.8 88.96) (end 162.76 88.96) (width 0.7) (layer F.Cu) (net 8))
 (segment (start 159.073655 98.96) (end 160.7 98.96) (width 0.7) (layer F.Cu) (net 8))
 (segment (start 150.08 88.96) (end 151.93 88.96) (width 0.7) (layer F.Cu) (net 8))
 (segment (start 147.53 91.51) (end 150.08 88.96) (width 0.7) (layer F.Cu) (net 8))
 (segment (start 145.33 91.51) (end 147.53 91.51) (width 0.7) (layer F.Cu) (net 8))
 (segment (start 151.93 88.96) (end 151.45 88.96) (width 0.7) (layer F.Cu) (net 8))
 (segment (start 157.2 90.16) (end 158.4 88.96) (width 0.7) (layer F.Cu) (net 8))
 (segment (start 157.2 97.66) (end 157.2 90.16) (width 0.7) (layer F.Cu) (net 8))
 (segment (start 158.5 98.96) (end 157.2 97.66) (width 0.7) (layer F.Cu) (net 8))
 (segment (start 160.7 98.96) (end 158.5 98.96) (width 0.7) (layer F.Cu) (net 8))
 (segment (start 160.5 88.96) (end 158.4 88.96) (width 0.7) (layer F.Cu) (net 8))
 (segment (start 158.4 88.96) (end 151.93 88.96) (width 0.7) (layer F.Cu) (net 8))
 (segment (start 160.4 78.9) (end 160.5 78.8) (width 0.7) (layer F.Cu) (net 8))
 (segment (start 156.8 78.8) (end 160.5 78.8) (width 0.7) (layer B.Cu) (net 8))
 (segment (start 145.33 89.27) (end 145.33 91.51) (width 0.7) (layer B.Cu) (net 8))
 (segment (start 160.5 78.8) (end 155.8 78.8) (width 0.7) (layer B.Cu) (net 8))
 (segment (start 155.8 78.8) (end 145.33 89.27) (width 0.7) (layer B.Cu) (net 8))
 (segment (start 121.35 86.45) (end 129.89 86.45) (width 0.7) (layer F.Cu) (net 3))
 (segment (start 99.244546 104.884532) (end 102.915468 104.884532) (width 0.7) (layer F.Cu) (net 3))
 (segment (start 102.915468 104.884532) (end 121.35 86.45) (width 0.7) (layer F.Cu) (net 3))
 (segment (start 127.184546 102.334532) (end 125.384546 102.334532) (width 0.7) (layer B.Cu) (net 2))
 (segment (start 91.699692 82.62501) (end 91.1 82.025318) (width 0.7) (layer B.Cu) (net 2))
 (segment (start 90.24 79.04) (end 88.26 79.04) (width 0.7) (layer B.Cu) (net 2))
 (segment (start 91.1 82.025318) (end 91.1 79.9) (width 0.7) (layer B.Cu) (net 2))
 (segment (start 91.1 79.9) (end 90.24 79.04) (width 0.7) (layer B.Cu) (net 2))
 (segment (start 91.699692 82.62501) (end 91.72501 82.62501) (width 0.7) (layer B.Cu) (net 2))
 (segment (start 92 82.9) (end 105.950014 82.9) (width 0.7) (layer B.Cu) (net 2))
 (segment (start 91.72501 82.62501) (end 92 82.9) (width 0.7) (layer B.Cu) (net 2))
 (segment (start 125.384546 102.334532) (end 105.950014 82.9) (width 0.7) (layer B.Cu) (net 2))
 (segment (start 125.384546 104.874532) (end 127.184546 104.874532) (width 0.7) (layer B.Cu) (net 1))
 (segment (start 88.26 81.58) (end 88.36 81.58) (width 0.7) (layer B.Cu) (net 1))
 (segment (start 88.36 81.58) (end 90.40502 83.62502) (width 0.7) (layer B.Cu) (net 1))
 (segment (start 90.42502 83.62502) (end 90.70001 83.90001) (width 0.7) (layer B.Cu) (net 1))
 (segment (start 90.40502 83.62502) (end 90.42502 83.62502) (width 0.7) (layer B.Cu) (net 1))
 (segment (start 90.70001 83.90001) (end 104.410024 83.90001) (width 0.7) (layer B.Cu) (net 1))
 (segment (start 104.410024 83.90001) (end 125.384546 104.874532) (width 0.7) (layer B.Cu) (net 1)))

